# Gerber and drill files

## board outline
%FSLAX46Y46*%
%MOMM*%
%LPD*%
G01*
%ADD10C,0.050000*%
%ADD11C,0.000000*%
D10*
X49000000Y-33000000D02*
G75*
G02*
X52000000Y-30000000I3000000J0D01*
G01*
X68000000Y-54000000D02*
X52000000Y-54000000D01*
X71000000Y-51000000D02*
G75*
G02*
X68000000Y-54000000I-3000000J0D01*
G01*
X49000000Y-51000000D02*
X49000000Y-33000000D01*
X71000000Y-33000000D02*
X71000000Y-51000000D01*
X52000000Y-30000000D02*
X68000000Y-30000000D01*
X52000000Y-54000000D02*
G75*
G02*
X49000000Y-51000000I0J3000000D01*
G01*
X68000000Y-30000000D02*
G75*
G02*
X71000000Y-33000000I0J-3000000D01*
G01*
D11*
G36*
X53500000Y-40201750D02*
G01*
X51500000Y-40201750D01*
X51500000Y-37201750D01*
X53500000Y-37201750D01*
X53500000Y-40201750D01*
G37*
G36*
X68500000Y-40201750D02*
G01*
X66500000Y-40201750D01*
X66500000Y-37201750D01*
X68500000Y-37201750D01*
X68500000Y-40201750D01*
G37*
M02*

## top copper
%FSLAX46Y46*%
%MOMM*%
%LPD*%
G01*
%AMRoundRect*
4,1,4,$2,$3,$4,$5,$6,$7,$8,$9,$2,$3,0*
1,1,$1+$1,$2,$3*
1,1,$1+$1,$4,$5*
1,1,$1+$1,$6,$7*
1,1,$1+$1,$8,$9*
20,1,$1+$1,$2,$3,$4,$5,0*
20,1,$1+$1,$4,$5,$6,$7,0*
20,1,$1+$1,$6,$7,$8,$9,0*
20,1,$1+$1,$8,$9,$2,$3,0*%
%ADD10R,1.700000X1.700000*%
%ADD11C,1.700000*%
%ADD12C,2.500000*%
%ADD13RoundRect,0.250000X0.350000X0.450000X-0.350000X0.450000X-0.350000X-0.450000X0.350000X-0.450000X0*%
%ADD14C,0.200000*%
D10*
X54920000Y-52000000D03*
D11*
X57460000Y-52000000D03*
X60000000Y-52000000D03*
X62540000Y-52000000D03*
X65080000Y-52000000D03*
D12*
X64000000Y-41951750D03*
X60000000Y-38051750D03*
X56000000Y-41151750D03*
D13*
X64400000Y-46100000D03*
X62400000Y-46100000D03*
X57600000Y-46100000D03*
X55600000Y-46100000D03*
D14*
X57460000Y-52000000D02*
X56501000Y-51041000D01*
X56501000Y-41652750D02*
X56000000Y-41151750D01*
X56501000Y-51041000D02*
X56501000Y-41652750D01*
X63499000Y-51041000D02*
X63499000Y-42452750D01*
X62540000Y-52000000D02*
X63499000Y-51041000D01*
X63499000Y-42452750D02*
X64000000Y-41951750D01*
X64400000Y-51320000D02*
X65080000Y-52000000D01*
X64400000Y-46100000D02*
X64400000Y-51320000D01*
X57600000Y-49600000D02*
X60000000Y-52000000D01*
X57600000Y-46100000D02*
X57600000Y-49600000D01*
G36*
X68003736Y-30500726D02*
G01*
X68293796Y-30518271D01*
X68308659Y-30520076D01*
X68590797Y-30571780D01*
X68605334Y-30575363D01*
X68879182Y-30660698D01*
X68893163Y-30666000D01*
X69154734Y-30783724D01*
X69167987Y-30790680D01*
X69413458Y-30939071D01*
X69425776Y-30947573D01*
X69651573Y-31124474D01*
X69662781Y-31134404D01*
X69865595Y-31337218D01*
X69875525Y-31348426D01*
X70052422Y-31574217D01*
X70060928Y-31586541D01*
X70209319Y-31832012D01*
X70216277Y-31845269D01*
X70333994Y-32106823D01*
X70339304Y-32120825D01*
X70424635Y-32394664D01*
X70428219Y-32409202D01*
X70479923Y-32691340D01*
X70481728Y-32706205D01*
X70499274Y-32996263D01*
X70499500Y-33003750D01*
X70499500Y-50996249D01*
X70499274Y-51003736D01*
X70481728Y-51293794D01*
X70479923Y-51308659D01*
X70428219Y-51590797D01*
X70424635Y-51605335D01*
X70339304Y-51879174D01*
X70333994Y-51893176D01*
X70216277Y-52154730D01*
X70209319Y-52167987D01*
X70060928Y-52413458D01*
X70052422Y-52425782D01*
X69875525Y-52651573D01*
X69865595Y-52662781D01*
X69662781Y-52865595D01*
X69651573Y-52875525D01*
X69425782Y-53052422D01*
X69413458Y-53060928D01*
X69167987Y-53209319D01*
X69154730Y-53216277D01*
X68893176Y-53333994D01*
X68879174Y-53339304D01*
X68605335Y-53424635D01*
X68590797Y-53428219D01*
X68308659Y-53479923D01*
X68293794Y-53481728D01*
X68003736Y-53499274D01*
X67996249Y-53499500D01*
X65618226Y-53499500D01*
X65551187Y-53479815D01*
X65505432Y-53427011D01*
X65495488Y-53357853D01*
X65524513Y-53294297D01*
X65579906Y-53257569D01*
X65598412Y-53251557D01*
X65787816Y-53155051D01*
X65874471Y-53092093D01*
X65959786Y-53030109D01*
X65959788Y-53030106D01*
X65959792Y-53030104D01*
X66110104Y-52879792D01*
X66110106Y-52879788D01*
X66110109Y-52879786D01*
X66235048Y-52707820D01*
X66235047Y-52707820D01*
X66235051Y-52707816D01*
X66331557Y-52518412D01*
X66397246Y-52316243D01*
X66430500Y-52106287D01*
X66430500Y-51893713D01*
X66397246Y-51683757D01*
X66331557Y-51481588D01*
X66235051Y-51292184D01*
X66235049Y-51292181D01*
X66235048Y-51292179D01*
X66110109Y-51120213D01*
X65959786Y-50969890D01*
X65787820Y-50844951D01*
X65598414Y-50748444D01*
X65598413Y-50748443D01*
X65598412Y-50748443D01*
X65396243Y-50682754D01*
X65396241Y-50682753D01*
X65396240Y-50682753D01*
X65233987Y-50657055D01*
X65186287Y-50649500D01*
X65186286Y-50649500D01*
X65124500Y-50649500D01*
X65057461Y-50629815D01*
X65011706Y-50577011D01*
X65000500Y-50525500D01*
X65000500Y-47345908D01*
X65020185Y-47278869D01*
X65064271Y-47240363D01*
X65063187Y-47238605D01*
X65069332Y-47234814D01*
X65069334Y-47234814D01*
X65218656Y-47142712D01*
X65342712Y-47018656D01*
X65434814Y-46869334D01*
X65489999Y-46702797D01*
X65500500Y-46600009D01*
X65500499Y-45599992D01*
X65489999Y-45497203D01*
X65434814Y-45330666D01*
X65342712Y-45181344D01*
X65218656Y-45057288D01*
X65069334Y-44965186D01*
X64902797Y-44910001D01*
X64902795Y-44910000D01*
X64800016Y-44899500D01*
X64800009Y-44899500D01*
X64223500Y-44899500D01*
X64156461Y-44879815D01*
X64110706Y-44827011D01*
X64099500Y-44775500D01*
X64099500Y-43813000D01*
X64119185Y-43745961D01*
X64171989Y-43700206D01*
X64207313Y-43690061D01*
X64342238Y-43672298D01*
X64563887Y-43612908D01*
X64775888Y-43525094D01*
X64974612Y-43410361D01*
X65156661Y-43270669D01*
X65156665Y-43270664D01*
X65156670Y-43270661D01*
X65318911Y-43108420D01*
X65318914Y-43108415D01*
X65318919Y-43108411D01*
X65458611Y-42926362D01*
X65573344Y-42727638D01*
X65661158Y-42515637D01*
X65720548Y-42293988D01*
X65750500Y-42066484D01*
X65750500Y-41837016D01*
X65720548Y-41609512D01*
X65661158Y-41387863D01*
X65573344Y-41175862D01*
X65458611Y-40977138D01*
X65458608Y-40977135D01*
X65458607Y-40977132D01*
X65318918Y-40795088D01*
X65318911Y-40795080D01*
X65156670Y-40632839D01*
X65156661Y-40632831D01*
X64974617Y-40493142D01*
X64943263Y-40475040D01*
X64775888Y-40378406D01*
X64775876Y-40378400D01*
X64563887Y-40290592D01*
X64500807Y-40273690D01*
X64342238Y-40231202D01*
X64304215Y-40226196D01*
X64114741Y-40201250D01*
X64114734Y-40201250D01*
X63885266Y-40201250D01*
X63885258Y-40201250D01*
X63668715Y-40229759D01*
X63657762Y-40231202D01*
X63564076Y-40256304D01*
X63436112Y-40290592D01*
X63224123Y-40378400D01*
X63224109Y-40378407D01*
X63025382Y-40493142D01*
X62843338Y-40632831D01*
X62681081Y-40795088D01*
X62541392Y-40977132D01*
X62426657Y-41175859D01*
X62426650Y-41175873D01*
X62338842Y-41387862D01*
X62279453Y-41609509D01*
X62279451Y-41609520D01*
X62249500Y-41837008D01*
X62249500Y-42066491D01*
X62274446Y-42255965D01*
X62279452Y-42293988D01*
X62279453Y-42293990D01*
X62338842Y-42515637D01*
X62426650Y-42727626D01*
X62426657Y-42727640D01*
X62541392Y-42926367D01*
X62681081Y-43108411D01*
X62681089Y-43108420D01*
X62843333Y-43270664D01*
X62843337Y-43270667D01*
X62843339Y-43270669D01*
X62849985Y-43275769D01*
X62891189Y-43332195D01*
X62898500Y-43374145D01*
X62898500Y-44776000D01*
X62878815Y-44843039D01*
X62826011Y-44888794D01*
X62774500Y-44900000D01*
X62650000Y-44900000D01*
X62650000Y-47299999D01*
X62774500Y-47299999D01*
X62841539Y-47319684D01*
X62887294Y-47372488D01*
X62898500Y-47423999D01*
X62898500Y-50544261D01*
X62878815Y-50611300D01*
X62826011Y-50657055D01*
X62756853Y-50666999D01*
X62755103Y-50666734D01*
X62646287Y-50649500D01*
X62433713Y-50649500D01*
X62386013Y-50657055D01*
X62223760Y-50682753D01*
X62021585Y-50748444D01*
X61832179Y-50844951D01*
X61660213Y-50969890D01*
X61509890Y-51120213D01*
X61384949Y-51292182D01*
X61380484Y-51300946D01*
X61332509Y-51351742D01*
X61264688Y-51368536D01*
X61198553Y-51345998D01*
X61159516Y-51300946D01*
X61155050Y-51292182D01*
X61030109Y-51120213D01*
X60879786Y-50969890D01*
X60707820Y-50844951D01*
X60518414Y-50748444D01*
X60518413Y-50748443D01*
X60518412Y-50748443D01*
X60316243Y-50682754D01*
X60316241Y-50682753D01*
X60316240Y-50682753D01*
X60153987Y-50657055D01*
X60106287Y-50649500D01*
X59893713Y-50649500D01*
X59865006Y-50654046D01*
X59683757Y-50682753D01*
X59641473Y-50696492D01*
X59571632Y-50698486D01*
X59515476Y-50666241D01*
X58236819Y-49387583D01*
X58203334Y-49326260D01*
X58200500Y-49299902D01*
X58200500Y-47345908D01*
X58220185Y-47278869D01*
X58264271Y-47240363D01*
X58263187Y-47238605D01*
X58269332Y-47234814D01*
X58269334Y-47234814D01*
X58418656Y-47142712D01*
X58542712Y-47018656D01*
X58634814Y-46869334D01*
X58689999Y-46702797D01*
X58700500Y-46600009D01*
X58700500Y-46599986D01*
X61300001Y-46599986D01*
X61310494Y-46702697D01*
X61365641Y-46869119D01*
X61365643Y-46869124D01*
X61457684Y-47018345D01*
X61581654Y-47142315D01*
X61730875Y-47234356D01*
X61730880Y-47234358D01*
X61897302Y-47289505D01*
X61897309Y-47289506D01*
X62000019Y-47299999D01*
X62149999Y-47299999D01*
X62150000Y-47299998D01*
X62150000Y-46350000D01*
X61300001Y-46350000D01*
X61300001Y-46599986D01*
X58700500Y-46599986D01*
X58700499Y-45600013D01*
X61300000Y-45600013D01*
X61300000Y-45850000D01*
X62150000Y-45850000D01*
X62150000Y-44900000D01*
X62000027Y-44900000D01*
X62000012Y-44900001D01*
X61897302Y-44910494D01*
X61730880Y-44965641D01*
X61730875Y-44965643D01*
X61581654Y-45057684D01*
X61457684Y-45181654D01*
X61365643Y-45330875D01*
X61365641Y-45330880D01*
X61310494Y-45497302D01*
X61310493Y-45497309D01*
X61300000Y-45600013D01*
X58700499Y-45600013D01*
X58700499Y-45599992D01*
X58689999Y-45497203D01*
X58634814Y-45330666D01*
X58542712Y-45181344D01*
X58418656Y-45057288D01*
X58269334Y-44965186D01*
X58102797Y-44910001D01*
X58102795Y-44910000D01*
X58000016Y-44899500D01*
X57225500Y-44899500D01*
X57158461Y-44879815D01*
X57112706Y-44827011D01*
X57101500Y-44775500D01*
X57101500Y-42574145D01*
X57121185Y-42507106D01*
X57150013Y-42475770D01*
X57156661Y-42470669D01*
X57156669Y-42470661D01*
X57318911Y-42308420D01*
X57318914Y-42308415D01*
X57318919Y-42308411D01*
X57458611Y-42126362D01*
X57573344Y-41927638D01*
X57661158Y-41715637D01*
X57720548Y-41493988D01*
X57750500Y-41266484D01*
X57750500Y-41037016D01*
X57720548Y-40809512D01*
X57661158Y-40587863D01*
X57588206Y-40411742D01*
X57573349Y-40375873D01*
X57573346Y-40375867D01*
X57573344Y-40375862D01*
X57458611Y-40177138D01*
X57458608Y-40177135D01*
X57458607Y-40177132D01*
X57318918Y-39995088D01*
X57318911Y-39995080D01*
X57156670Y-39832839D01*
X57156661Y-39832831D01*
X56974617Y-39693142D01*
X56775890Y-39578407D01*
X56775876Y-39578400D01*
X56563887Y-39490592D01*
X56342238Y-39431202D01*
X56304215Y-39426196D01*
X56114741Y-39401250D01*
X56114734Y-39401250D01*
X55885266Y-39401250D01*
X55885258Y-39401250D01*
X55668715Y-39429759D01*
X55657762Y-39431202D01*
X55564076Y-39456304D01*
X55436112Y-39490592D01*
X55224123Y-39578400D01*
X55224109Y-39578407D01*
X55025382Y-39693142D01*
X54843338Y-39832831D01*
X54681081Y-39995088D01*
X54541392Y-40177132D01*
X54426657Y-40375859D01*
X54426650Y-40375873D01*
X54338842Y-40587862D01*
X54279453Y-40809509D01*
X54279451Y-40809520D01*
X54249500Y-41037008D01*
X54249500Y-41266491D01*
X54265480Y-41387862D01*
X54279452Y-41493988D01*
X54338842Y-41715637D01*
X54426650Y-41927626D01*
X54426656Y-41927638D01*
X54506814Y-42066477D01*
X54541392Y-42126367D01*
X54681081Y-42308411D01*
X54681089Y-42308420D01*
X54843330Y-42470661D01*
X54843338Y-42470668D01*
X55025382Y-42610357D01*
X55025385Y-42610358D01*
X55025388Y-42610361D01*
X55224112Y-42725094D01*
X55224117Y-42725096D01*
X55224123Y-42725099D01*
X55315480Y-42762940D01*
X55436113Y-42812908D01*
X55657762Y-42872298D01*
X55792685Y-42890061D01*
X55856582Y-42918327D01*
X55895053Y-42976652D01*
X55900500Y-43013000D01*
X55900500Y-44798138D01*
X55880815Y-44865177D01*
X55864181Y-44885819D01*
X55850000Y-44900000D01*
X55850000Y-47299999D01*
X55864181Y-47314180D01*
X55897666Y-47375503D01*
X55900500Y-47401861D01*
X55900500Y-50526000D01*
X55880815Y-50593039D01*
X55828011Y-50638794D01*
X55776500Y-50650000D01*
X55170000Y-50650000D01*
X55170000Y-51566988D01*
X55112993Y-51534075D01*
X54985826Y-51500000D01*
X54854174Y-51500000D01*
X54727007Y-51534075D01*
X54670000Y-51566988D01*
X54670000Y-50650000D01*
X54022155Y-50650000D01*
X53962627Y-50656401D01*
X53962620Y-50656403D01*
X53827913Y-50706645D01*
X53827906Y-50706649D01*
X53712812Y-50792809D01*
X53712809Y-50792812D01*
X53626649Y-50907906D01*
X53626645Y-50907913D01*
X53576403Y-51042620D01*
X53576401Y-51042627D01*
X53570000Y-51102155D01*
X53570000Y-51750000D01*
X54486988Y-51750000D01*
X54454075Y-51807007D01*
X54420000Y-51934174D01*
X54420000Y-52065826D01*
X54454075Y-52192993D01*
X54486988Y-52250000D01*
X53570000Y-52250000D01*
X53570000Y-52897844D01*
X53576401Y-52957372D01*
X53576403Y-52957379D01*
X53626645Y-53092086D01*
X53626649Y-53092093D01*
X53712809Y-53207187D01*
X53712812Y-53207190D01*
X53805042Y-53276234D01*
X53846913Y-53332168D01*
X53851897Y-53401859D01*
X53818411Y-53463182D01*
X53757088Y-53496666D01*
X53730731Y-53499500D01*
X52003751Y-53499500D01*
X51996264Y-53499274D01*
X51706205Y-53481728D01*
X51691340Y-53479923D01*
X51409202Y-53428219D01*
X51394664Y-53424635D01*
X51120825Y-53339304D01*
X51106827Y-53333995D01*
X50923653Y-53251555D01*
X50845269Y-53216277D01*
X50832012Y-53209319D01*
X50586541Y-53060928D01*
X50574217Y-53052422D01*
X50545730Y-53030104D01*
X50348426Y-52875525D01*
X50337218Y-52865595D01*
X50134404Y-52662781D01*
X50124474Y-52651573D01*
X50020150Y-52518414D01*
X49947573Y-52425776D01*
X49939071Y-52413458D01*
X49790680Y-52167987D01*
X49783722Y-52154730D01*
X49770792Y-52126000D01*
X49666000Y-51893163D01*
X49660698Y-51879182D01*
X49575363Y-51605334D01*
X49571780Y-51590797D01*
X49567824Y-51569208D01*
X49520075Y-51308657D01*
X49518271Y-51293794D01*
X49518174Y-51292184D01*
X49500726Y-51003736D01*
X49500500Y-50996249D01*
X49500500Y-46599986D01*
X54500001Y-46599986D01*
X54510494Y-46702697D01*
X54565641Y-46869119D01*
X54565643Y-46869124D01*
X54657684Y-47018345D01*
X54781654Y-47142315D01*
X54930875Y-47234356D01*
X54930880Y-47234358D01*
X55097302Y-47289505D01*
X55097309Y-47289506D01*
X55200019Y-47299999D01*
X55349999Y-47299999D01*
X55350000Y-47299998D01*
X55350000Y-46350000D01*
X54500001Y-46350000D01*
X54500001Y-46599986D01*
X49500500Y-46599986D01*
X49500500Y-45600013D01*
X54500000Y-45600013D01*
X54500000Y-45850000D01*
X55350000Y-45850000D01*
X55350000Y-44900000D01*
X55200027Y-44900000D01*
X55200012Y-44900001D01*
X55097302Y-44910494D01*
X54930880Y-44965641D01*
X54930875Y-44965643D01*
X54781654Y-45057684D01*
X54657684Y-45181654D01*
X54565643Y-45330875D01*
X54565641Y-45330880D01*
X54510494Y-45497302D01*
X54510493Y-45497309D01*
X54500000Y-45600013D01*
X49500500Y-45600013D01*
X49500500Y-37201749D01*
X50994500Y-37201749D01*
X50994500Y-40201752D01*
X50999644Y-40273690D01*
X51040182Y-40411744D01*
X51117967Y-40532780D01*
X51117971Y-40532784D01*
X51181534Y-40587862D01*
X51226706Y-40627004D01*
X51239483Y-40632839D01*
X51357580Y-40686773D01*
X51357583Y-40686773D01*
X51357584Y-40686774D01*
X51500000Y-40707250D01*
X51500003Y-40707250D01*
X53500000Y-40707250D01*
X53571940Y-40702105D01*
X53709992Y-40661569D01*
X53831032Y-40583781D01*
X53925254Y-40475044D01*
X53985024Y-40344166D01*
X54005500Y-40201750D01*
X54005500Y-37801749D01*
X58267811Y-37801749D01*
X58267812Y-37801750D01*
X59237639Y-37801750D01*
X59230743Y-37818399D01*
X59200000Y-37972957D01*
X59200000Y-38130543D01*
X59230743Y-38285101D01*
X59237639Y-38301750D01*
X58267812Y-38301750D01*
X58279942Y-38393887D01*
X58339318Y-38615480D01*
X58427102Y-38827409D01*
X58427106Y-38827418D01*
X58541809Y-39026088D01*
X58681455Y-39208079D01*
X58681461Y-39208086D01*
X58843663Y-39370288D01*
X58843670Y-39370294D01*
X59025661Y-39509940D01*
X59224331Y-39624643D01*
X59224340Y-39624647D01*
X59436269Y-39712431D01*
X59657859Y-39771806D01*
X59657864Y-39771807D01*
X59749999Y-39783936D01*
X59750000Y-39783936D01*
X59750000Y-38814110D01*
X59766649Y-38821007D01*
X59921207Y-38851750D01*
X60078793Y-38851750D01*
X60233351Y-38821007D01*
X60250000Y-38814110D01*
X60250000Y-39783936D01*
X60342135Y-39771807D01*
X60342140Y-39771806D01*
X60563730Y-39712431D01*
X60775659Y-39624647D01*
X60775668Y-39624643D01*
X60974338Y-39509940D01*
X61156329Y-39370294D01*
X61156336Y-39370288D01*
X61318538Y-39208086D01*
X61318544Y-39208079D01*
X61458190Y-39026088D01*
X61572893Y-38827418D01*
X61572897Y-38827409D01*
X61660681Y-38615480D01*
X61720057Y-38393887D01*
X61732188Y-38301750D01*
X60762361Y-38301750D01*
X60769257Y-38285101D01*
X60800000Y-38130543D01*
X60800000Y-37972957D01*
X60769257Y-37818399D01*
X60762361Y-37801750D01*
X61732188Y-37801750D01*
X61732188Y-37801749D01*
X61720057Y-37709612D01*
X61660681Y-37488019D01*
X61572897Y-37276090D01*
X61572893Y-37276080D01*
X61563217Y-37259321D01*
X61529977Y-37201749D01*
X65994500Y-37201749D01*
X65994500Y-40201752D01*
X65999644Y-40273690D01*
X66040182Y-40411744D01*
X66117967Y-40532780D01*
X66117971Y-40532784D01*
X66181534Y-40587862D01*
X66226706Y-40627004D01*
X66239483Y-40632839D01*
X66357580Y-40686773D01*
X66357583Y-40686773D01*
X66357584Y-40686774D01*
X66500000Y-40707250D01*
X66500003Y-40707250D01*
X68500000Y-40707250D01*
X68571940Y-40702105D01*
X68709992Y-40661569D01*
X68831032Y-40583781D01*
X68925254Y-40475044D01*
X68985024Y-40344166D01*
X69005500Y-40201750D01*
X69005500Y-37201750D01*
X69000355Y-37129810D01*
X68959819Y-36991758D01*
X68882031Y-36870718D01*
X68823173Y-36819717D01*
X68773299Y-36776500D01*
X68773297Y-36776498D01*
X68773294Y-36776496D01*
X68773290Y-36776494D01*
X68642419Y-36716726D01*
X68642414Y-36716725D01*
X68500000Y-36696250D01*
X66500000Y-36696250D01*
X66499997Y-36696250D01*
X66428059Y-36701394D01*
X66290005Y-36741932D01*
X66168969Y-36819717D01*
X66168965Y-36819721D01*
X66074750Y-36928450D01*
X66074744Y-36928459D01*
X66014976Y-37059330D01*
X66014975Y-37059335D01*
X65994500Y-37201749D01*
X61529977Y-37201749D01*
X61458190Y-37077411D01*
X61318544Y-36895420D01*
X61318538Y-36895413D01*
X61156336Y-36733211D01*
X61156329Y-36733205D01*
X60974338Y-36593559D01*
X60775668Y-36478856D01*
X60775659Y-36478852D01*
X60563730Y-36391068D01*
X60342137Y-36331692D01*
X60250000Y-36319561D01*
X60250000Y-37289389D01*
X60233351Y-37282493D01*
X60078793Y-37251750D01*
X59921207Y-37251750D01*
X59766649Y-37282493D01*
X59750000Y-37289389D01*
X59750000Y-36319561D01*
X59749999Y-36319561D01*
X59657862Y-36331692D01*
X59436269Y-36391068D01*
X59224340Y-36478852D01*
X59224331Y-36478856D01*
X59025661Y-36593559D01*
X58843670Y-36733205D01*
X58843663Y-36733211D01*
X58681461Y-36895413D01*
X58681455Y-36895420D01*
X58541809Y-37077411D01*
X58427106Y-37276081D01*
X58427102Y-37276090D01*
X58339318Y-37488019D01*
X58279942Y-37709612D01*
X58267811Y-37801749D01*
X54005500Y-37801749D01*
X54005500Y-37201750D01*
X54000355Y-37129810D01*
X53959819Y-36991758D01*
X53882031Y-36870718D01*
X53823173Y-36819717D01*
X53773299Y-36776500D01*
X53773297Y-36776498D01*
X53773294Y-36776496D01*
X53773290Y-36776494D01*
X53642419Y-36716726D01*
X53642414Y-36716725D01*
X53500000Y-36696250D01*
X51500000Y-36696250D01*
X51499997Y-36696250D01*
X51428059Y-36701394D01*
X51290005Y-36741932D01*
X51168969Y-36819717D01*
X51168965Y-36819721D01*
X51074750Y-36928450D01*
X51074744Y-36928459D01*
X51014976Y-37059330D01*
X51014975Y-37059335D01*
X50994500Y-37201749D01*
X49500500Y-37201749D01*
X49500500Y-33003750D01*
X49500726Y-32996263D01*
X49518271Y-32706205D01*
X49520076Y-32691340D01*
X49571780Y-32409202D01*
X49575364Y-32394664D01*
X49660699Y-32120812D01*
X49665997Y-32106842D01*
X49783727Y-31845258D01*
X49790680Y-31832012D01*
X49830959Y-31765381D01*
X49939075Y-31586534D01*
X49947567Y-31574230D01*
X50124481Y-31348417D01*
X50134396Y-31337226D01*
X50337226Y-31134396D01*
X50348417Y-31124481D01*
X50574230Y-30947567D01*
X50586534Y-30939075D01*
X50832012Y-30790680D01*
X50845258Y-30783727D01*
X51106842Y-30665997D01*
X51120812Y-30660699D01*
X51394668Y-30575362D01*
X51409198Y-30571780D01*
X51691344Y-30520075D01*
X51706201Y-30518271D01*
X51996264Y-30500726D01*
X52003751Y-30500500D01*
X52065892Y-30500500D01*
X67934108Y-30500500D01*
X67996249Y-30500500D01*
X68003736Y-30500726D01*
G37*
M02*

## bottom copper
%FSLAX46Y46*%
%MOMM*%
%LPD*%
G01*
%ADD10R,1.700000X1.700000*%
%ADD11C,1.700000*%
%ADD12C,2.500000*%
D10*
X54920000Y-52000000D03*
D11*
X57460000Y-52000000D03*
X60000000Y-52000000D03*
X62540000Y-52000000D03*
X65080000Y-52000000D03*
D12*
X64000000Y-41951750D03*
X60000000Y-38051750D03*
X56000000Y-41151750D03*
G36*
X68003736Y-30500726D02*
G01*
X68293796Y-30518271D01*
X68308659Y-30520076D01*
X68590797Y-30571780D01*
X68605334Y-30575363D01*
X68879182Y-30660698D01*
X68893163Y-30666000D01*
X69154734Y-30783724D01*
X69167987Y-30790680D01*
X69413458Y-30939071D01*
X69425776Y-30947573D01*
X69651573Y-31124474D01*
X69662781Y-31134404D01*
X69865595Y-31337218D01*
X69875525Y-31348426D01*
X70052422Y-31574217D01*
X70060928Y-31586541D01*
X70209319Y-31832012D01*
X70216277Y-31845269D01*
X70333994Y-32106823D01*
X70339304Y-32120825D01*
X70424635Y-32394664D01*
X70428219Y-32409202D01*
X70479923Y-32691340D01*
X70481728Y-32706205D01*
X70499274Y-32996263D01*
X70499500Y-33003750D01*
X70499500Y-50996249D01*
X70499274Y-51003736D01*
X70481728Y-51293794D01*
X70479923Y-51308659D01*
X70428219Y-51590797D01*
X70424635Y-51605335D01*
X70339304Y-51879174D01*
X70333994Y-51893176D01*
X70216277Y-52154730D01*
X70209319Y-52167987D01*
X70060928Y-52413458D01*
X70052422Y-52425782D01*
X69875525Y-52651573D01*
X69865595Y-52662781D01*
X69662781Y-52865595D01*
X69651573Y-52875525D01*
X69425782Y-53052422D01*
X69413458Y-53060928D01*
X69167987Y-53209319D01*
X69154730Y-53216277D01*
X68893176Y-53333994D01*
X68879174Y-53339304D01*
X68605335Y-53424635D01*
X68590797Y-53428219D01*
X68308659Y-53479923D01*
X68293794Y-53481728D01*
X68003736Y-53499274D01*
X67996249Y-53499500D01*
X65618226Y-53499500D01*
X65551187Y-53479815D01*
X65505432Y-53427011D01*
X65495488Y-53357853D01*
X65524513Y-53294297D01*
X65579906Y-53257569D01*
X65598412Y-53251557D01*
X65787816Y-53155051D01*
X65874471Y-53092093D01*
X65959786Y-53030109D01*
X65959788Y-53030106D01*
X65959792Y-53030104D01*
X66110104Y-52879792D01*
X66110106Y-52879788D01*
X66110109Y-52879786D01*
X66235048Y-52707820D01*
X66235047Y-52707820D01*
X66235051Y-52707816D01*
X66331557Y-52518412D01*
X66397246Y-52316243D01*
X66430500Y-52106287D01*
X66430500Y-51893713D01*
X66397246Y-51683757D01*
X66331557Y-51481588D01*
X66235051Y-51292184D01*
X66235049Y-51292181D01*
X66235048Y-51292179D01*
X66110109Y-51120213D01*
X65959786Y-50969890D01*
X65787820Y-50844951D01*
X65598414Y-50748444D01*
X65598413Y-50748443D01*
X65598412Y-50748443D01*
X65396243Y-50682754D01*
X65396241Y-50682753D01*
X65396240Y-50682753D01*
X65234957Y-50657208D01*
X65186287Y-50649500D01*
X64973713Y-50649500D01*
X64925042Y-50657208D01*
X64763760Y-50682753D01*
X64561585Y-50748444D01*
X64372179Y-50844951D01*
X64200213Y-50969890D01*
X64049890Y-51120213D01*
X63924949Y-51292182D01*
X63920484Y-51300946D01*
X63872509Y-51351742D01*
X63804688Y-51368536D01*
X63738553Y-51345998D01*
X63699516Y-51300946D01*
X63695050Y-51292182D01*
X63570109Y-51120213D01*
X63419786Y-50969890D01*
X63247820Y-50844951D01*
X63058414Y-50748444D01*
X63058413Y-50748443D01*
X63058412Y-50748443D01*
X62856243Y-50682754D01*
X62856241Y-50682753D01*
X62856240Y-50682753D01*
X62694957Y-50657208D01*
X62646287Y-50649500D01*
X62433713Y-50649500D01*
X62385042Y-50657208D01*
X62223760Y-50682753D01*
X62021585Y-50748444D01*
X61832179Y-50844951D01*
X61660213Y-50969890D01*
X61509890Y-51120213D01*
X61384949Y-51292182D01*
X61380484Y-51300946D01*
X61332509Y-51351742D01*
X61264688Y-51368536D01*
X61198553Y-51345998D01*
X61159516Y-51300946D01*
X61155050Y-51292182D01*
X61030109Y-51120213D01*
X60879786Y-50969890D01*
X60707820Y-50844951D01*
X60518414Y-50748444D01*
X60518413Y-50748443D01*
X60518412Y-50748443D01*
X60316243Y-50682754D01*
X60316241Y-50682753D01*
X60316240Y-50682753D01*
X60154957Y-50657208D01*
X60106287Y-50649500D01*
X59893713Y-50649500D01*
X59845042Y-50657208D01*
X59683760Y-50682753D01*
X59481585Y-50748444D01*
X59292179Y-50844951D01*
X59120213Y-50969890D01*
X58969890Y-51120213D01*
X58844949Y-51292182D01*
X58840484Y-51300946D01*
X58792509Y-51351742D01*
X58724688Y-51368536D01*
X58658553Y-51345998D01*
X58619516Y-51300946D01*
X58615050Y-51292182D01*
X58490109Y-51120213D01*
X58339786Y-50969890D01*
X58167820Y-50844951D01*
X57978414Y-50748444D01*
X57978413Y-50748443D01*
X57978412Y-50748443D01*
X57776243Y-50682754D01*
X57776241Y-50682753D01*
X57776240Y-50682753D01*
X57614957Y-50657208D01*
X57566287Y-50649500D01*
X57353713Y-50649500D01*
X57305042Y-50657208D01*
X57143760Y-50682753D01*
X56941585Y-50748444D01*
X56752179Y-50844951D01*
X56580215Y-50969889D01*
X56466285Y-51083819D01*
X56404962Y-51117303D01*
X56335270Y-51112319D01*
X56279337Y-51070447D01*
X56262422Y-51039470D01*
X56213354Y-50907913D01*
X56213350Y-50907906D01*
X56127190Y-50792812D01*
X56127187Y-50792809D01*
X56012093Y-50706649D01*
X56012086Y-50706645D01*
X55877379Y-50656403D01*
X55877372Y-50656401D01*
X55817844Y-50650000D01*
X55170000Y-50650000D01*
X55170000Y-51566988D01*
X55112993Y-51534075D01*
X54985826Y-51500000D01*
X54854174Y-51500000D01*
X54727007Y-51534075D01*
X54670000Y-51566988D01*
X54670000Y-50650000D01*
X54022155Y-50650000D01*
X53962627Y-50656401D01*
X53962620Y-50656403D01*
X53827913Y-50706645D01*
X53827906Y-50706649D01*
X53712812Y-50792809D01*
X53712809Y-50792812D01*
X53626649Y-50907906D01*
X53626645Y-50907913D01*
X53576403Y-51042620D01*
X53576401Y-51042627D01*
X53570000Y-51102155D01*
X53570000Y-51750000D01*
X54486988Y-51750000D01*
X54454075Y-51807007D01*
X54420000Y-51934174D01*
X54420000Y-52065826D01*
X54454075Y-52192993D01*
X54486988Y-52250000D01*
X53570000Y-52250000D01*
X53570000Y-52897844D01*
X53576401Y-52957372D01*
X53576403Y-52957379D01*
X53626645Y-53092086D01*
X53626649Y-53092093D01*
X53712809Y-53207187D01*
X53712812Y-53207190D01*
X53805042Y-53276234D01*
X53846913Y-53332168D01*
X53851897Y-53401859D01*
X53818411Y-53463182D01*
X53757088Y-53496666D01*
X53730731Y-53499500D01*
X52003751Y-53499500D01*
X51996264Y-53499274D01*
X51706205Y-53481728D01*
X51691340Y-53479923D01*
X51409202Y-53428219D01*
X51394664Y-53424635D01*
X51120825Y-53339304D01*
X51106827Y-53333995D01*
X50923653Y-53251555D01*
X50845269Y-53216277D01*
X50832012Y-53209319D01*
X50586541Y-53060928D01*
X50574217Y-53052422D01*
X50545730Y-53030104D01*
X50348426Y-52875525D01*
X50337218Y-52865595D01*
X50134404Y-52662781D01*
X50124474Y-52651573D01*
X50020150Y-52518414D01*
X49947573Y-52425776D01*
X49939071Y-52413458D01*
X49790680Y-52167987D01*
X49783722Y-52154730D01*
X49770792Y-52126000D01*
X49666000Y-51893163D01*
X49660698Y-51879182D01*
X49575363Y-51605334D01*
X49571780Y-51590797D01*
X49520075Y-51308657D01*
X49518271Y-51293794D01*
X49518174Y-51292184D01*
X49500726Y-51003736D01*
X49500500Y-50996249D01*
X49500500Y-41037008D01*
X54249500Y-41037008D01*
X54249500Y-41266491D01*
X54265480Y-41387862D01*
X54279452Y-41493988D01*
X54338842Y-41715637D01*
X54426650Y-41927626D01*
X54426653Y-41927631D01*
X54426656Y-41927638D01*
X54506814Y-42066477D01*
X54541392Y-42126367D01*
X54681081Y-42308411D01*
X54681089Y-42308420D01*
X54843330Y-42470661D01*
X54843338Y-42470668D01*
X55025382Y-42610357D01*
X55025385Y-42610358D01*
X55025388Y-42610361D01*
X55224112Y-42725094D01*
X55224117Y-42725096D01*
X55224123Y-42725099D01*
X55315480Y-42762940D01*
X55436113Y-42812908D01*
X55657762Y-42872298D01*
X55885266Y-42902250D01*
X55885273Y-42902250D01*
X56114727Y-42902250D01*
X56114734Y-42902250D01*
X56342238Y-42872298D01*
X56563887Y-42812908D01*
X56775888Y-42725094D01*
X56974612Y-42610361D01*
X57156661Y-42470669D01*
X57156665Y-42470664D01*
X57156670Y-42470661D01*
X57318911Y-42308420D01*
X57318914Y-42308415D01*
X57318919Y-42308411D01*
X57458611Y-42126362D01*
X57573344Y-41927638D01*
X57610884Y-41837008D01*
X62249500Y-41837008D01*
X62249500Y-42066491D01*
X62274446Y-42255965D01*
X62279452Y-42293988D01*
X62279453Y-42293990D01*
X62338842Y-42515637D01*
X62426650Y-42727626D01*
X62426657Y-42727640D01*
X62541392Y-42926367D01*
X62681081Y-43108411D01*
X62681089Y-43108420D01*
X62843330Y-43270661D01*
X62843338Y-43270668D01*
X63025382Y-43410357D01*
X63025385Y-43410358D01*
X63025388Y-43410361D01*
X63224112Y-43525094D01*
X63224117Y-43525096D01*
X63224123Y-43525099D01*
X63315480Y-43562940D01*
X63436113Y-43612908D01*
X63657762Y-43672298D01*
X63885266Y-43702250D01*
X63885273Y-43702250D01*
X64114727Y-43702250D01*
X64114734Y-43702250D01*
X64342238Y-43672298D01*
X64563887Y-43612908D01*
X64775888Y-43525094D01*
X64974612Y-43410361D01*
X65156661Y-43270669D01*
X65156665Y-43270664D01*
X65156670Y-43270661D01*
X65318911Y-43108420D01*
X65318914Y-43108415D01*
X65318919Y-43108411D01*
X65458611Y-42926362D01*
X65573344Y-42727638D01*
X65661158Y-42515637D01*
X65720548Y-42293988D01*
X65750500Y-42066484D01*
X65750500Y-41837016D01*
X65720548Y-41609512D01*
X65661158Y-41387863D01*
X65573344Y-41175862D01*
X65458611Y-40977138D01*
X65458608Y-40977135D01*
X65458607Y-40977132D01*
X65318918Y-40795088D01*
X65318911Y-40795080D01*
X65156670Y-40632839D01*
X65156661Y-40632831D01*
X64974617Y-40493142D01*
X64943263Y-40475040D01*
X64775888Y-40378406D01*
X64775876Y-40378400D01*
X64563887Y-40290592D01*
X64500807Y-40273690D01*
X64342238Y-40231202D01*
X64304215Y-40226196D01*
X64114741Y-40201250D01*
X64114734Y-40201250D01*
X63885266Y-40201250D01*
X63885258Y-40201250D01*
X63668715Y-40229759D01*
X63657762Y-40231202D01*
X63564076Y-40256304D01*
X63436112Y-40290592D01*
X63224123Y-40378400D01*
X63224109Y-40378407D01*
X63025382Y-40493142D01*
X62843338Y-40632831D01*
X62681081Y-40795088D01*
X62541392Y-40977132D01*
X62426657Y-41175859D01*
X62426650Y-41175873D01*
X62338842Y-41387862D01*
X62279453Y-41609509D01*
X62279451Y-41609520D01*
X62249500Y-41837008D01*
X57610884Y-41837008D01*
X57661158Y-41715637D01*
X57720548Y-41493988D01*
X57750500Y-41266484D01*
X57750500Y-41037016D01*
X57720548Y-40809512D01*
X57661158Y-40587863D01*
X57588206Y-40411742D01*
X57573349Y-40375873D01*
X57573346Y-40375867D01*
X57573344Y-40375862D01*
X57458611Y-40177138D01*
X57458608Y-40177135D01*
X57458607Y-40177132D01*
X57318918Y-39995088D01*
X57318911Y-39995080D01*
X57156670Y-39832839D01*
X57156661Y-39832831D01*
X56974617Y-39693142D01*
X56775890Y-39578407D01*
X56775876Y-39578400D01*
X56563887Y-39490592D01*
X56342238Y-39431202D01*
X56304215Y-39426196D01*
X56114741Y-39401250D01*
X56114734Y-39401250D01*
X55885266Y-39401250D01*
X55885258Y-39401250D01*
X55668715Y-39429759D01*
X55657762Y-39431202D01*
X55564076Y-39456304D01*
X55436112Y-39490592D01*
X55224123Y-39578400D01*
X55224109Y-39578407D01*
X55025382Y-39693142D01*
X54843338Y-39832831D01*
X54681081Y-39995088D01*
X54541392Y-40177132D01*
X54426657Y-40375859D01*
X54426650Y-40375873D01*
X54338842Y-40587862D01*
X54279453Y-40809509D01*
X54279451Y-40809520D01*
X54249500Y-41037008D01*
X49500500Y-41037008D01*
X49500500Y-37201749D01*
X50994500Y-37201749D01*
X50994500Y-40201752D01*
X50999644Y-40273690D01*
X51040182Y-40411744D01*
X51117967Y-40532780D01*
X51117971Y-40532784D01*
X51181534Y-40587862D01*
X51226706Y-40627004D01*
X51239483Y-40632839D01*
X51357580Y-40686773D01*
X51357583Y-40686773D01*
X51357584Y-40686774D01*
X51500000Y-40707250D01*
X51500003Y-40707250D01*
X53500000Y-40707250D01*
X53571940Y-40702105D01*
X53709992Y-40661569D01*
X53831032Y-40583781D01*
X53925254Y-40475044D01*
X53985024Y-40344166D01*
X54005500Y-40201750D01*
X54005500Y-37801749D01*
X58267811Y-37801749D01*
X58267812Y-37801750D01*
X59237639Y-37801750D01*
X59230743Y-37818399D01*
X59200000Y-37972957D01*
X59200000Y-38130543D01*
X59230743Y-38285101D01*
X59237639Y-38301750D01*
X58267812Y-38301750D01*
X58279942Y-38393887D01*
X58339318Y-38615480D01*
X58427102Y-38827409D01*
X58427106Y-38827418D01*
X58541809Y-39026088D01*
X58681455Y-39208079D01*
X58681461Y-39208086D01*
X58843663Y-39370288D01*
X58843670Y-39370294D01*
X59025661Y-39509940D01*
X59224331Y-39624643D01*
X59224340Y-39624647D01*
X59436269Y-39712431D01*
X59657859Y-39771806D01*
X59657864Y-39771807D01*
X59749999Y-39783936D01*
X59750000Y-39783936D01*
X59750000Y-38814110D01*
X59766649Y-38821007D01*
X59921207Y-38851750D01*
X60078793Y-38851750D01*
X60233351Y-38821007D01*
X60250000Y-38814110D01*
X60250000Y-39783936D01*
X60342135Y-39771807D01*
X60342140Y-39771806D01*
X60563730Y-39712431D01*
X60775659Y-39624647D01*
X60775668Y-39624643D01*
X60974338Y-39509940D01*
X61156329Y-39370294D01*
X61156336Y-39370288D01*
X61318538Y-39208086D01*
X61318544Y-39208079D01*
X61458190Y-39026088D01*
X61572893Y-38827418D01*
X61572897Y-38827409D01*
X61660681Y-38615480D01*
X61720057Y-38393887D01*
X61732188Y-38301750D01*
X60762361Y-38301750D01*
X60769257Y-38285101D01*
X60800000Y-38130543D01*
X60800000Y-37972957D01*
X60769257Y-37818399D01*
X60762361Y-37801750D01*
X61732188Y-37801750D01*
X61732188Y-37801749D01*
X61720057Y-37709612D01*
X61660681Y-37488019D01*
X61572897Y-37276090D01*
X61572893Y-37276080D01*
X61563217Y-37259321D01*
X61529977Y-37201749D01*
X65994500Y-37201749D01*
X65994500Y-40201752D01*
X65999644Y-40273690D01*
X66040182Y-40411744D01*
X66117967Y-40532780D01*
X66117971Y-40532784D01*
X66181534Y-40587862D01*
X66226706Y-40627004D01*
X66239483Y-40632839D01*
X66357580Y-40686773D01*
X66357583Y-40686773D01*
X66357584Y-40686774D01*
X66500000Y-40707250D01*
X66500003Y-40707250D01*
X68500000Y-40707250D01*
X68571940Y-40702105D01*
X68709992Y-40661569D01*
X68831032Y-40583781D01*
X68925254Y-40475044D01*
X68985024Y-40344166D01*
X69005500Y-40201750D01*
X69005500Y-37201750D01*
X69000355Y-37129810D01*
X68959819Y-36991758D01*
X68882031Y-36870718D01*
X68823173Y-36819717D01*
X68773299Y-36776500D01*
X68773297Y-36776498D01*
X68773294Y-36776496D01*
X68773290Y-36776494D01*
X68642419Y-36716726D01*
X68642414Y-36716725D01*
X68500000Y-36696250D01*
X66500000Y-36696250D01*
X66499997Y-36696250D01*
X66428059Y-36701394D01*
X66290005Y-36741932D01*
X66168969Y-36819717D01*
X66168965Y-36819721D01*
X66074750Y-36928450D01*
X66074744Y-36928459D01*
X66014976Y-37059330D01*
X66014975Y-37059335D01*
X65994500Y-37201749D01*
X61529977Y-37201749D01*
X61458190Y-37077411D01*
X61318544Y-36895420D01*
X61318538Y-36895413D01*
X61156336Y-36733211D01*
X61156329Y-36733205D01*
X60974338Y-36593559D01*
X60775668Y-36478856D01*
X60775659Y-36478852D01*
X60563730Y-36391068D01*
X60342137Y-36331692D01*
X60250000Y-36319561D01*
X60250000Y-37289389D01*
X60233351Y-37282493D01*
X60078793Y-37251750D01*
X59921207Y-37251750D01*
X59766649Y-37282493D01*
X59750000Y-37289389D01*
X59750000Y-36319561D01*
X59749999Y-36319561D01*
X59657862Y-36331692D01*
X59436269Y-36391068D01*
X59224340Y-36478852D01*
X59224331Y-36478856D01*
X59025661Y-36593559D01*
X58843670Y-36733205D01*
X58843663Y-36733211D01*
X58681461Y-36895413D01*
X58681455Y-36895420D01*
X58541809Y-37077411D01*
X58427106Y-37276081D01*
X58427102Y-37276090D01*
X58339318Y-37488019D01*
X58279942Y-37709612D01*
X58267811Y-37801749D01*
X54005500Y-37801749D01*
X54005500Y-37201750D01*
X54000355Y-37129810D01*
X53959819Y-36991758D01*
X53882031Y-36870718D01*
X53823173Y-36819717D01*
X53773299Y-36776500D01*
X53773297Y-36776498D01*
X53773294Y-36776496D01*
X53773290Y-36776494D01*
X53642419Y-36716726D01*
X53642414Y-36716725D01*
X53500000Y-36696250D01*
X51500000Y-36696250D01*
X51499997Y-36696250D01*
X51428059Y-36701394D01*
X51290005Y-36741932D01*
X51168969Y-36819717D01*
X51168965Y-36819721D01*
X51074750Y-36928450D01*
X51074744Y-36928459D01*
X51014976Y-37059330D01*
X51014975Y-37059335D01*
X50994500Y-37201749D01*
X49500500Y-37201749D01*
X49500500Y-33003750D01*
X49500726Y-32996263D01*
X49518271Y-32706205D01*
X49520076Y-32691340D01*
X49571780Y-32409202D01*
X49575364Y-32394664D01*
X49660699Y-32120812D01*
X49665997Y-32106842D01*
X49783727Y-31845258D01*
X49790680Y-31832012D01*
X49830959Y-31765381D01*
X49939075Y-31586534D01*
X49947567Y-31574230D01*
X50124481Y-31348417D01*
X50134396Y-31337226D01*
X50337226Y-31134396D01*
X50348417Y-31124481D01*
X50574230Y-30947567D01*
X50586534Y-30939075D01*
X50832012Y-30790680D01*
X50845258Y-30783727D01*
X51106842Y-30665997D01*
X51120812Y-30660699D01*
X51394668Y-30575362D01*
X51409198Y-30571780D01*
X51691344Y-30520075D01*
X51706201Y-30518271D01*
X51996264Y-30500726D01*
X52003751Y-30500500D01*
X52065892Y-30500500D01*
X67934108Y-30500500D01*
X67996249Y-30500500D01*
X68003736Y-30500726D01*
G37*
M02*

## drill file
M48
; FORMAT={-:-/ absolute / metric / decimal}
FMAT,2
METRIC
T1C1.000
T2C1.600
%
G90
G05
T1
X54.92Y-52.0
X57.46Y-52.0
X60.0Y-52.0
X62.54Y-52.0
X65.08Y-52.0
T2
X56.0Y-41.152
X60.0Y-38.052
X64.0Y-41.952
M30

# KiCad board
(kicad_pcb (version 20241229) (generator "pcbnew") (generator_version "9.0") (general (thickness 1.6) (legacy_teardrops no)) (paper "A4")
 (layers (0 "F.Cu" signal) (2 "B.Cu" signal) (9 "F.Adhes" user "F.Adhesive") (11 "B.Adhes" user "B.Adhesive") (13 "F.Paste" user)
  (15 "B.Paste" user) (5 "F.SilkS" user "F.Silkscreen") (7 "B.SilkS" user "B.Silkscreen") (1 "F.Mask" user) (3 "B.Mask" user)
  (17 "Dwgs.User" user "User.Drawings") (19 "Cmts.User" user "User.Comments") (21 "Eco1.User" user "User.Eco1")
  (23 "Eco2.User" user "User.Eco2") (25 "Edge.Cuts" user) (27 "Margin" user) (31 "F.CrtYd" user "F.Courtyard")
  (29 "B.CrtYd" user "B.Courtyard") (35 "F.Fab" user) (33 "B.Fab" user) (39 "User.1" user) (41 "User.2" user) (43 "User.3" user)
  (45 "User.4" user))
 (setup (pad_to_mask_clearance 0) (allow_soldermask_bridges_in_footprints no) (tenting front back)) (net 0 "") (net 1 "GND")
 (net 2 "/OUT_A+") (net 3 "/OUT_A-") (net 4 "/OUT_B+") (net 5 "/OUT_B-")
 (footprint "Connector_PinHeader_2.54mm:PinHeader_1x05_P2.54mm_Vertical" (layer "F.Cu") (at 54.92 52 90)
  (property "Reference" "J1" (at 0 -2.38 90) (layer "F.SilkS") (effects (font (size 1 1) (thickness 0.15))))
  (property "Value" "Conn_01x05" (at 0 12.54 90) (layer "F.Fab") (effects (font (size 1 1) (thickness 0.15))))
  (pad "1" thru_hole rect (at 0 0 90) (size 1.7 1.7) (drill 1) (layers "*.Cu" "*.Mask") (remove_unused_layers no) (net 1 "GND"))
  (pad "2" thru_hole circle (at 0 2.54 90) (size 1.7 1.7) (drill 1) (layers "*.Cu" "*.Mask") (remove_unused_layers no) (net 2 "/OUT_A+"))
  (pad "3" thru_hole circle (at 0 5.08 90) (size 1.7 1.7) (drill 1) (layers "*.Cu" "*.Mask") (remove_unused_layers no) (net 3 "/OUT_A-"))
  (pad "4" thru_hole circle (at 0 7.62 90) (size 1.7 1.7) (drill 1) (layers "*.Cu" "*.Mask") (remove_unused_layers no) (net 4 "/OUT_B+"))
  (pad "5" thru_hole circle (at 0 10.16 90) (size 1.7 1.7) (drill 1) (layers "*.Cu" "*.Mask") (remove_unused_layers no) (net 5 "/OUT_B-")))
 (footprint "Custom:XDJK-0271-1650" (layer "F.Cu") (at 60 40.00175 180)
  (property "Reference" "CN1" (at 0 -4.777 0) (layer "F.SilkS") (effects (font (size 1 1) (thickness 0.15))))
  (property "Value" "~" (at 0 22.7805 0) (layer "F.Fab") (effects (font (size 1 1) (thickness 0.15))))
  (fp_poly (pts (xy 6.5 2.8) (xy 6.5 -0.2) (xy 8.5 -0.2) (xy 8.5 2.8)) (stroke (width 0) (type default)) (fill yes) (layer "Edge.Cuts"))
  (fp_poly (pts (xy -8.5 2.8) (xy -8.5 -0.2) (xy -6.5 -0.2) (xy -6.5 2.8)) (stroke (width 0) (type default)) (fill yes) (layer "Edge.Cuts"))
  (pad "1" thru_hole circle (at -4 -1.95 180) (size 2.5 2.5) (drill 1.6) (layers "*.Cu" "*.Mask") (remove_unused_layers no)
   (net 4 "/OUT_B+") (thermal_bridge_angle 90))
  (pad "2" thru_hole circle (at 0 1.95 180) (size 2.5 2.5) (drill 1.6) (layers "*.Cu" "*.Mask") (remove_unused_layers no) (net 1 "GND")
   (thermal_bridge_angle 90))
  (pad "3" thru_hole circle (at 4 -1.15 180) (size 2.5 2.5) (drill 1.6) (layers "*.Cu" "*.Mask") (remove_unused_layers no) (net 2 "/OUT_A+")
   (thermal_bridge_angle 90)))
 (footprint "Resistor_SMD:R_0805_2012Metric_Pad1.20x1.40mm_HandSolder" (layer "F.Cu") (at 63.4 46.1 180)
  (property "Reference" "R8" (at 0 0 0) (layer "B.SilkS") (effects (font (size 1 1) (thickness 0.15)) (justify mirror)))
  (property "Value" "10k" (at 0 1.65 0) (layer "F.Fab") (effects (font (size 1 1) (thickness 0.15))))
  (pad "1" smd roundrect (at -1 0 180) (size 1.2 1.4) (layers "F.Cu" "F.Mask" "F.Paste") (roundrect_rratio 0.208333) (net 5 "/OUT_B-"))
  (pad "2" smd roundrect (at 1 0 180) (size 1.2 1.4) (layers "F.Cu" "F.Mask" "F.Paste") (roundrect_rratio 0.208333) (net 1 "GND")))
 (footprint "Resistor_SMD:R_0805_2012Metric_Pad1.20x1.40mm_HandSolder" (layer "F.Cu") (at 56.6 46.1 180)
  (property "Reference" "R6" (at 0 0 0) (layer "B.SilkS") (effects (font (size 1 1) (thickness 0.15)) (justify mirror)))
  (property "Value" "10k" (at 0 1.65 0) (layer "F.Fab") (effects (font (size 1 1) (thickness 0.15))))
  (pad "1" smd roundrect (at -1 0 180) (size 1.2 1.4) (layers "F.Cu" "F.Mask" "F.Paste") (roundrect_rratio 0.208333) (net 3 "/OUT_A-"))
  (pad "2" smd roundrect (at 1 0 180) (size 1.2 1.4) (layers "F.Cu" "F.Mask" "F.Paste") (roundrect_rratio 0.208333) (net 1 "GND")))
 (gr_arc (start 49 33) (mid 49.87868 30.87868) (end 52 30) (stroke (width 0.05) (type default)) (layer "Edge.Cuts"))
 (gr_line (start 68 54) (end 52 54) (stroke (width 0.05) (type default)) (layer "Edge.Cuts"))
 (gr_arc (start 71 51) (mid 70.12132 53.12132) (end 68 54) (stroke (width 0.05) (type default)) (layer "Edge.Cuts"))
 (gr_line (start 49 51) (end 49 33) (stroke (width 0.05) (type default)) (layer "Edge.Cuts"))
 (gr_line (start 71 33) (end 71 51) (stroke (width 0.05) (type default)) (layer "Edge.Cuts"))
 (gr_line (start 52 30) (end 68 30) (stroke (width 0.05) (type default)) (layer "Edge.Cuts"))
 (gr_arc (start 52 54) (mid 49.87868 53.12132) (end 49 51) (stroke (width 0.05) (type default)) (layer "Edge.Cuts"))
 (gr_arc (start 68 30) (mid 70.12132 30.87868) (end 71 33) (stroke (width 0.05) (type default)) (layer "Edge.Cuts"))
 (segment (start 57.46 52) (end 56.501 51.041) (width 0.2) (layer "F.Cu") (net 2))
 (segment (start 56.501 41.65275) (end 56 41.15175) (width 0.2) (layer "F.Cu") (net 2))
 (segment (start 56.501 51.041) (end 56.501 41.65275) (width 0.2) (layer "F.Cu") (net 2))
 (segment (start 63.499 51.041) (end 63.499 42.45275) (width 0.2) (layer "F.Cu") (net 4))
 (segment (start 62.54 52) (end 63.499 51.041) (width 0.2) (layer "F.Cu") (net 4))
 (segment (start 63.499 42.45275) (end 64 41.95175) (width 0.2) (layer "F.Cu") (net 4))
 (segment (start 64.4 51.32) (end 65.08 52) (width 0.2) (layer "F.Cu") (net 5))
 (segment (start 64.4 46.1) (end 64.4 51.32) (width 0.2) (layer "F.Cu") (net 5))
 (segment (start 57.6 49.6) (end 60 52) (width 0.2) (layer "F.Cu") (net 3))
 (segment (start 57.6 46.1) (end 57.6 49.6) (width 0.2) (layer "F.Cu") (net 3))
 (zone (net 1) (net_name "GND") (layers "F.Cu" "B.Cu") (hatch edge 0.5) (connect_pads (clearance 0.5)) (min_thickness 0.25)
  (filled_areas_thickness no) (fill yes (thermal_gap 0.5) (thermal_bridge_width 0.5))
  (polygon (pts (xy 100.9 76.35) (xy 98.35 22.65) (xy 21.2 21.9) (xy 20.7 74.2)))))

